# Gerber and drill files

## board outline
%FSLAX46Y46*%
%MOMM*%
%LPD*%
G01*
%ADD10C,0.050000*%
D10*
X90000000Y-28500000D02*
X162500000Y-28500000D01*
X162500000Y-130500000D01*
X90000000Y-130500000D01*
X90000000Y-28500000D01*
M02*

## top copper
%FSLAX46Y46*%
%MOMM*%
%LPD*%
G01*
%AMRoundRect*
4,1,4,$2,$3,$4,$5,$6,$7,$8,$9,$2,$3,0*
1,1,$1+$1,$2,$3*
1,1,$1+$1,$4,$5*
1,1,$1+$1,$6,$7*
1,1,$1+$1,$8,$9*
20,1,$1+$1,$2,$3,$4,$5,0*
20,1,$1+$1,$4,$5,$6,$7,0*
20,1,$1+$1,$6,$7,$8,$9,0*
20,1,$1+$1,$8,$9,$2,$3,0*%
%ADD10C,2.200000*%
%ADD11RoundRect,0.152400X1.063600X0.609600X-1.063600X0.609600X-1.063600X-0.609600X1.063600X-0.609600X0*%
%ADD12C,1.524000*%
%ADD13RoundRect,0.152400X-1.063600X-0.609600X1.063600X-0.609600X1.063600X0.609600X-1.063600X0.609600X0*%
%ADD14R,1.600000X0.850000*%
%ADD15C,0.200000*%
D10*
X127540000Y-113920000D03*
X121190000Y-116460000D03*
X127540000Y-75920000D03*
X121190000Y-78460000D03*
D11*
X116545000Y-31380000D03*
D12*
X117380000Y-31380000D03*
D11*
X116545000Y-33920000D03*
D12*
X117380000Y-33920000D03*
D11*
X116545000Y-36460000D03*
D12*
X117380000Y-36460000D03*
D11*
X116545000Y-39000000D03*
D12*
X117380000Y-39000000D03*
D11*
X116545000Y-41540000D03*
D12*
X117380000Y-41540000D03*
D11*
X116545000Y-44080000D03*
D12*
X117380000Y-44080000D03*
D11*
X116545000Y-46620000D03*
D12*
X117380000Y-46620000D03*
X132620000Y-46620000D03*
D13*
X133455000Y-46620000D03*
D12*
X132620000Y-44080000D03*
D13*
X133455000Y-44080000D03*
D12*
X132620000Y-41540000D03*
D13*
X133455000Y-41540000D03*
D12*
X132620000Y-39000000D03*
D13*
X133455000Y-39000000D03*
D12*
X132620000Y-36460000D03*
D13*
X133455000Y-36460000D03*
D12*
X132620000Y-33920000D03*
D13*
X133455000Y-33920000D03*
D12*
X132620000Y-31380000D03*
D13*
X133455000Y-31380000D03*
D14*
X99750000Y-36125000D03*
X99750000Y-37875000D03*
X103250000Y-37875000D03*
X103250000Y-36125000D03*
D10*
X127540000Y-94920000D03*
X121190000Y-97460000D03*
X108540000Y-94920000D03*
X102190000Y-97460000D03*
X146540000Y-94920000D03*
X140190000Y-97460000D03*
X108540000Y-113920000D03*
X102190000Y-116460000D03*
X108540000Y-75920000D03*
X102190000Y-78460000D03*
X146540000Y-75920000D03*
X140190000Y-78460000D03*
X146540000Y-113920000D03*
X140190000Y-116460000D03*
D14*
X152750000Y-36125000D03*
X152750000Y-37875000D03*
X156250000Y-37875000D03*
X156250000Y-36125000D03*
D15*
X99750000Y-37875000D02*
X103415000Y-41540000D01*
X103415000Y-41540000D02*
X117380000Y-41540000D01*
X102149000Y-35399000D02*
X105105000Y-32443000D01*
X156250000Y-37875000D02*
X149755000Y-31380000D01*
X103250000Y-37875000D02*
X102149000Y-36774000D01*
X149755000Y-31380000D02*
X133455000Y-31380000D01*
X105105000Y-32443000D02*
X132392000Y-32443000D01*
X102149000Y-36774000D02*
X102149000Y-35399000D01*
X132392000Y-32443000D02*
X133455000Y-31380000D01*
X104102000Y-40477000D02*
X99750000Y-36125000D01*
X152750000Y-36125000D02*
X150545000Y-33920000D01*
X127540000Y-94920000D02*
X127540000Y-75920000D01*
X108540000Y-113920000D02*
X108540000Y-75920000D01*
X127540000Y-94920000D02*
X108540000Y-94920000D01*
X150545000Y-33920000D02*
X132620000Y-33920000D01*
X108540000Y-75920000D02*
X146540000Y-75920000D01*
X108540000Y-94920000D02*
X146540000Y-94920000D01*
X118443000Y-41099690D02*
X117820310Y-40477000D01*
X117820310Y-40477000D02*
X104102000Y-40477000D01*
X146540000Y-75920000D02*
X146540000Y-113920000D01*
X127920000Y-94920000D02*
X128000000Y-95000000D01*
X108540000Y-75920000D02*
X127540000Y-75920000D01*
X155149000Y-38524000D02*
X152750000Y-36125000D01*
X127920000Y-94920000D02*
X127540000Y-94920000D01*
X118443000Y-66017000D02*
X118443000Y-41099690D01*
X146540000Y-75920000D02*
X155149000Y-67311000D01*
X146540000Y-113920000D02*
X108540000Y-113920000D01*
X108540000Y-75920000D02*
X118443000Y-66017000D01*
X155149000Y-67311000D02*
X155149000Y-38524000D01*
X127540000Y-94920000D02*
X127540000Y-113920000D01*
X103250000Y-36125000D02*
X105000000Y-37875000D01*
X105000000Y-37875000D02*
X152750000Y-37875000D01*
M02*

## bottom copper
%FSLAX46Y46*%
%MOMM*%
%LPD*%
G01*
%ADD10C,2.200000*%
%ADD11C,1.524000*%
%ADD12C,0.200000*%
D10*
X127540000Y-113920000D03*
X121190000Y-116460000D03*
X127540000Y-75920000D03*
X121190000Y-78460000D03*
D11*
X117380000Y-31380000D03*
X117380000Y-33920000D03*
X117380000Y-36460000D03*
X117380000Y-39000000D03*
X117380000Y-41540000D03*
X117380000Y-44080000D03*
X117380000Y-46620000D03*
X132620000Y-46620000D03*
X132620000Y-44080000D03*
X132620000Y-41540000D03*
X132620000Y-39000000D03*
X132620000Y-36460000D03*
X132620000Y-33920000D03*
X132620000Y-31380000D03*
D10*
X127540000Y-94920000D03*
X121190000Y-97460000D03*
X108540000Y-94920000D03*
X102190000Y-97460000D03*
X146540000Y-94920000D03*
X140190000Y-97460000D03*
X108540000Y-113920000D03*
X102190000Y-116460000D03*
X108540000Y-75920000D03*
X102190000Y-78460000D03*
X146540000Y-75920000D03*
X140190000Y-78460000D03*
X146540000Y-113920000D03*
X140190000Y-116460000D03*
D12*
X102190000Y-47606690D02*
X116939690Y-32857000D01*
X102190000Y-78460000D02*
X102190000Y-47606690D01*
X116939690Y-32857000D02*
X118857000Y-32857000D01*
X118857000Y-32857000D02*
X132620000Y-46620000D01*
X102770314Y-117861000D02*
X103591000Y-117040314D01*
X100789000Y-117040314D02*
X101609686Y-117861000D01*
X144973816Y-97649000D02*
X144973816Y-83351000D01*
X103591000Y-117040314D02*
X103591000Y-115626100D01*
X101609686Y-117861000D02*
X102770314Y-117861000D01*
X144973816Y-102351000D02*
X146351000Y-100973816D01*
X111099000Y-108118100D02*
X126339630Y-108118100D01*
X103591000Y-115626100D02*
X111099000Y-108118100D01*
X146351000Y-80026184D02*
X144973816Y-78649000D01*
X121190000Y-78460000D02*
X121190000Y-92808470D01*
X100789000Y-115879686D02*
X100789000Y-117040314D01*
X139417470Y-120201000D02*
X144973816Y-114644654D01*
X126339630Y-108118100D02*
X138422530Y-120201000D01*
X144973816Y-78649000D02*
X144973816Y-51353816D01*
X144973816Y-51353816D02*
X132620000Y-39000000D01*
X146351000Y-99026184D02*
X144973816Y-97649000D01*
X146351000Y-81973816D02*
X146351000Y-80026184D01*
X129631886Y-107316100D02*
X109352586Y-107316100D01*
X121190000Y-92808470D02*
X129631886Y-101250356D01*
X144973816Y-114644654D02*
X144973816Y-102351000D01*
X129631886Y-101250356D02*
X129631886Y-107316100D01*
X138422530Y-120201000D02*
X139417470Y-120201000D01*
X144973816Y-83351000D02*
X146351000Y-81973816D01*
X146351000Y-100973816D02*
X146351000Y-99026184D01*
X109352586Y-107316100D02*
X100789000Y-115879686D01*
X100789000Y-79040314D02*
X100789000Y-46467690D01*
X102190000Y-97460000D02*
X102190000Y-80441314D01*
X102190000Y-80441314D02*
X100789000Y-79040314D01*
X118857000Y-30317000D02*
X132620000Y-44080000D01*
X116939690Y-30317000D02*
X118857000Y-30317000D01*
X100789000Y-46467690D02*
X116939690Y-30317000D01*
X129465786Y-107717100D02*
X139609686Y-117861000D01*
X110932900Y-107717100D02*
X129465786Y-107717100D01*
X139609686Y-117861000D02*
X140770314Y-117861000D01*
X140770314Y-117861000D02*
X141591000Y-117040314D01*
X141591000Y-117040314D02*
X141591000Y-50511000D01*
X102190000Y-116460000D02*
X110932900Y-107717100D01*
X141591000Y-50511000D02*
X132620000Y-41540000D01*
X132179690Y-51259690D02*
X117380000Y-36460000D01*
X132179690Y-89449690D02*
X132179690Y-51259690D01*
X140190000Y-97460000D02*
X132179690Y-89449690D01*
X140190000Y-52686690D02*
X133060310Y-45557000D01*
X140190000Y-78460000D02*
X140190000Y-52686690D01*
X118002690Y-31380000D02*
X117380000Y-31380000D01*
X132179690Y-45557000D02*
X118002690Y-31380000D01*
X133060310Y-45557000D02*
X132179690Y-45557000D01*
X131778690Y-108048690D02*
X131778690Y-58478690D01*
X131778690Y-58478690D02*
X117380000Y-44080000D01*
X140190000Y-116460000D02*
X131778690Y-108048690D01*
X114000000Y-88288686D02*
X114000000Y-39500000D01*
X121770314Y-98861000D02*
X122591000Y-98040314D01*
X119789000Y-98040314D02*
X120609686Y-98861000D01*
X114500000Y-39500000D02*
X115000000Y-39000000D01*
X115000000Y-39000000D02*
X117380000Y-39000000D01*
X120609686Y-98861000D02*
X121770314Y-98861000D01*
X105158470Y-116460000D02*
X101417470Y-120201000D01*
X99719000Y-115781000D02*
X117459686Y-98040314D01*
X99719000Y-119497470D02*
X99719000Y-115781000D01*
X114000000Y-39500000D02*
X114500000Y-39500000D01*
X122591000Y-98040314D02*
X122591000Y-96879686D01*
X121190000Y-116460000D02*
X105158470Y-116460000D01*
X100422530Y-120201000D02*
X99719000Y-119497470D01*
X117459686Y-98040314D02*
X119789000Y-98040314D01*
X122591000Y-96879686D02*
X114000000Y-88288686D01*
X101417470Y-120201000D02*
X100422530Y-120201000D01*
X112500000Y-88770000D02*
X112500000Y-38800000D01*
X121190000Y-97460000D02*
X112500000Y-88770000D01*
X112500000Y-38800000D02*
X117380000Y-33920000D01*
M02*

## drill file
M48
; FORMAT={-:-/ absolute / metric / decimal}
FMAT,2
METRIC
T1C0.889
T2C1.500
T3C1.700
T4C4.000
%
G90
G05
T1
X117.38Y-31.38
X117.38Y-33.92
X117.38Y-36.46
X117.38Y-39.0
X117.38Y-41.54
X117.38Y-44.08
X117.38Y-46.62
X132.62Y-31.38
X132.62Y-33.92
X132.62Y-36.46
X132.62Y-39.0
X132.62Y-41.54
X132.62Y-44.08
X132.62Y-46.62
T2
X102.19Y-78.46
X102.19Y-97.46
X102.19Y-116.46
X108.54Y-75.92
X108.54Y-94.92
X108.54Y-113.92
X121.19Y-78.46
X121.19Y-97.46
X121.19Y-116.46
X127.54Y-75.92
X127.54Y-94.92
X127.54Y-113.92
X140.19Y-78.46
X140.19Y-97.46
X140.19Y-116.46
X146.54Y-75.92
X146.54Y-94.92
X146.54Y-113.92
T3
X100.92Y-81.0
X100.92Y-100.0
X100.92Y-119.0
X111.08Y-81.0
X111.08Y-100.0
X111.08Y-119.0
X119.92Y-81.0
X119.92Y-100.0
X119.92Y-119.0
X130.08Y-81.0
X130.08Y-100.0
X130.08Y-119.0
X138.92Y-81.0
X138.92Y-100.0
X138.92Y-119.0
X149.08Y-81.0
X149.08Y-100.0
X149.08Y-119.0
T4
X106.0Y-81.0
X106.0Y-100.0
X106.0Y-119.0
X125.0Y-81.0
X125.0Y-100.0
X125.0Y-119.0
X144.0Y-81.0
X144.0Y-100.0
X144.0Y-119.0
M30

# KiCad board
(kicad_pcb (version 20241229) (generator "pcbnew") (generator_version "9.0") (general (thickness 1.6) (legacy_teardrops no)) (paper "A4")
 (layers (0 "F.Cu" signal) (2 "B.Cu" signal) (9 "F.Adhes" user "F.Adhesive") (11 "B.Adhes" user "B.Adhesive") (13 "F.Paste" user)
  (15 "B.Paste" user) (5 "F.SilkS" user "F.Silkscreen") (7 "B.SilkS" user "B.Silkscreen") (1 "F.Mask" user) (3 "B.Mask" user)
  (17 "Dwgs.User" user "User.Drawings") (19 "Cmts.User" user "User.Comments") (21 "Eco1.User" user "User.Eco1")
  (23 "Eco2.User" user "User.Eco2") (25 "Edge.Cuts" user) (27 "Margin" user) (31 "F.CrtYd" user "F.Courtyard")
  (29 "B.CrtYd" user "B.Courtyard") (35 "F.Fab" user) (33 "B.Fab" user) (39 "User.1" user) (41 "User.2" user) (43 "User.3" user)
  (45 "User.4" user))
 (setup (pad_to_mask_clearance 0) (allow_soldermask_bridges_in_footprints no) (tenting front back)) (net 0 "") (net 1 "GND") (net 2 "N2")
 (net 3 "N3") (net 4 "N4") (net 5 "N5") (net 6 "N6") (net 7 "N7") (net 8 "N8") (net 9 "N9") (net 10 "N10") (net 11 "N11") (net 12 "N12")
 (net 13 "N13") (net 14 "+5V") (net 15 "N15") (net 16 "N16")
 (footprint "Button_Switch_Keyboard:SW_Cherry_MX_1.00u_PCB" (layer "F.Cu") (at 127.54 113.92)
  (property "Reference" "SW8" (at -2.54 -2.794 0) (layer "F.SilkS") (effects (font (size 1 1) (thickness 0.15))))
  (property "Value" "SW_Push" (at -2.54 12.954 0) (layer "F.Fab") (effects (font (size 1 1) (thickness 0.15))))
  (pad "" np_thru_hole circle (at -7.62 5.08) (size 1.7 1.7) (drill 1.7) (layers "*.Cu" "*.Mask"))
  (pad "" np_thru_hole circle (at -2.54 5.08) (size 4 4) (drill 4) (layers "*.Cu" "*.Mask"))
  (pad "" np_thru_hole circle (at 2.54 5.08) (size 1.7 1.7) (drill 1.7) (layers "*.Cu" "*.Mask"))
  (pad "1" thru_hole circle (at 0 0) (size 2.2 2.2) (drill 1.5) (layers "*.Cu" "*.Mask") (remove_unused_layers no) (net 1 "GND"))
  (pad "2" thru_hole circle (at -6.35 2.54) (size 2.2 2.2) (drill 1.5) (layers "*.Cu" "*.Mask") (remove_unused_layers no) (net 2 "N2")))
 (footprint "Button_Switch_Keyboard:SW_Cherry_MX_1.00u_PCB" (layer "F.Cu") (at 127.54 75.92)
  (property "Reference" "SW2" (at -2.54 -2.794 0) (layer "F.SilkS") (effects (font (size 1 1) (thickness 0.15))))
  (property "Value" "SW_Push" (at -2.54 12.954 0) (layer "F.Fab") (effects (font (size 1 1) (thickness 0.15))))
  (pad "" np_thru_hole circle (at -7.62 5.08) (size 1.7 1.7) (drill 1.7) (layers "*.Cu" "*.Mask"))
  (pad "" np_thru_hole circle (at -2.54 5.08) (size 4 4) (drill 4) (layers "*.Cu" "*.Mask"))
  (pad "" np_thru_hole circle (at 2.54 5.08) (size 1.7 1.7) (drill 1.7) (layers "*.Cu" "*.Mask"))
  (pad "1" thru_hole circle (at 0 0) (size 2.2 2.2) (drill 1.5) (layers "*.Cu" "*.Mask") (remove_unused_layers no) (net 1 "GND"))
  (pad "2" thru_hole circle (at -6.35 2.54) (size 2.2 2.2) (drill 1.5) (layers "*.Cu" "*.Mask") (remove_unused_layers no) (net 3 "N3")))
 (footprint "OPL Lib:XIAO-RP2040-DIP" (layer "F.Cu") (at 125 39)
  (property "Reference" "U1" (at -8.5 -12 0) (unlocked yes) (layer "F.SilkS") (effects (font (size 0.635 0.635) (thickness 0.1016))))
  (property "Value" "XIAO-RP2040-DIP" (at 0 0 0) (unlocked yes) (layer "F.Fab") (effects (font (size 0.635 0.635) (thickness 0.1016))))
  (pad "1" smd roundrect (at -8.455 -7.62 180) (size 2.432 1.524) (layers "F.Cu" "F.Mask") (roundrect_rratio 0.1) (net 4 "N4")
   (thermal_bridge_angle 45))
  (pad "1" thru_hole circle (at -7.62 -7.62 180) (size 1.524 1.524) (drill 0.889) (layers "*.Cu" "*.Mask") (remove_unused_layers no)
   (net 4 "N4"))
  (pad "2" smd roundrect (at -8.455 -5.08 180) (size 2.432 1.524) (layers "F.Cu" "F.Mask") (roundrect_rratio 0.1) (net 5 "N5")
   (thermal_bridge_angle 45))
  (pad "2" thru_hole circle (at -7.62 -5.08 180) (size 1.524 1.524) (drill 0.889) (layers "*.Cu" "*.Mask") (remove_unused_layers no)
   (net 5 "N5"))
  (pad "3" smd roundrect (at -8.455 -2.54 180) (size 2.432 1.524) (layers "F.Cu" "F.Mask") (roundrect_rratio 0.1) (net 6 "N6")
   (thermal_bridge_angle 45))
  (pad "3" thru_hole circle (at -7.62 -2.54 180) (size 1.524 1.524) (drill 0.889) (layers "*.Cu" "*.Mask") (remove_unused_layers no)
   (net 6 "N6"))
  (pad "4" smd roundrect (at -8.455 0 180) (size 2.432 1.524) (layers "F.Cu" "F.Mask") (roundrect_rratio 0.1) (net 2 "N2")
   (thermal_bridge_angle 45))
  (pad "4" thru_hole circle (at -7.62 0 180) (size 1.524 1.524) (drill 0.889) (layers "*.Cu" "*.Mask") (remove_unused_layers no)
   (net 2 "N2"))
  (pad "5" smd roundrect (at -8.455 2.54 180) (size 2.432 1.524) (layers "F.Cu" "F.Mask") (roundrect_rratio 0.1) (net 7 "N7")
   (thermal_bridge_angle 45))
  (pad "5" thru_hole circle (at -7.62 2.54 180) (size 1.524 1.524) (drill 0.889) (layers "*.Cu" "*.Mask") (remove_unused_layers no)
   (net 7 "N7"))
  (pad "6" smd roundrect (at -8.455 5.08 180) (size 2.432 1.524) (layers "F.Cu" "F.Mask") (roundrect_rratio 0.1) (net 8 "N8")
   (thermal_bridge_angle 45))
  (pad "6" thru_hole circle (at -7.62 5.08 180) (size 1.524 1.524) (drill 0.889) (layers "*.Cu" "*.Mask") (remove_unused_layers no)
   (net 8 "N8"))
  (pad "7" smd roundrect (at -8.455 7.62 180) (size 2.432 1.524) (layers "F.Cu" "F.Mask") (roundrect_rratio 0.1) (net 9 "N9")
   (thermal_bridge_angle 45))
  (pad "7" thru_hole circle (at -7.62 7.62 180) (size 1.524 1.524) (drill 0.889) (layers "*.Cu" "*.Mask") (remove_unused_layers no)
   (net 9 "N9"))
  (pad "8" thru_hole circle (at 7.62 7.62) (size 1.524 1.524) (drill 0.889) (layers "*.Cu" "*.Mask") (remove_unused_layers no)
   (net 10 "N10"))
  (pad "8" smd roundrect (at 8.455 7.62) (size 2.432 1.524) (layers "F.Cu" "F.Mask") (roundrect_rratio 0.1) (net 10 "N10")
   (thermal_bridge_angle 45))
  (pad "9" thru_hole circle (at 7.62 5.08) (size 1.524 1.524) (drill 0.889) (layers "*.Cu" "*.Mask") (remove_unused_layers no)
   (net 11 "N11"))
  (pad "9" smd roundrect (at 8.455 5.08) (size 2.432 1.524) (layers "F.Cu" "F.Mask") (roundrect_rratio 0.1) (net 11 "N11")
   (thermal_bridge_angle 45))
  (pad "10" thru_hole circle (at 7.62 2.54) (size 1.524 1.524) (drill 0.889) (layers "*.Cu" "*.Mask") (remove_unused_layers no)
   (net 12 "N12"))
  (pad "10" smd roundrect (at 8.455 2.54) (size 2.432 1.524) (layers "F.Cu" "F.Mask") (roundrect_rratio 0.1) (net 12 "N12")
   (thermal_bridge_angle 45))
  (pad "11" thru_hole circle (at 7.62 0) (size 1.524 1.524) (drill 0.889) (layers "*.Cu" "*.Mask") (remove_unused_layers no) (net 3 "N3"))
  (pad "11" smd roundrect (at 8.455 0) (size 2.432 1.524) (layers "F.Cu" "F.Mask") (roundrect_rratio 0.1) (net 3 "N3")
   (thermal_bridge_angle 45))
  (pad "12" thru_hole circle (at 7.62 -2.54) (size 1.524 1.524) (drill 0.889) (layers "*.Cu" "*.Mask") (remove_unused_layers no)
   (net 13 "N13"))
  (pad "12" smd roundrect (at 8.455 -2.54) (size 2.432 1.524) (layers "F.Cu" "F.Mask") (roundrect_rratio 0.1) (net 13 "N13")
   (thermal_bridge_angle 45))
  (pad "13" thru_hole circle (at 7.62 -5.08) (size 1.524 1.524) (drill 0.889) (layers "*.Cu" "*.Mask") (remove_unused_layers no)
   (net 1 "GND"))
  (pad "13" smd roundrect (at 8.455 -5.08) (size 2.432 1.524) (layers "F.Cu" "F.Mask") (roundrect_rratio 0.1) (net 1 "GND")
   (thermal_bridge_angle 45))
  (pad "14" thru_hole circle (at 7.62 -7.62) (size 1.524 1.524) (drill 0.889) (layers "*.Cu" "*.Mask") (remove_unused_layers no)
   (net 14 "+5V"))
  (pad "14" smd roundrect (at 8.455 -7.62) (size 2.432 1.524) (layers "F.Cu" "F.Mask") (roundrect_rratio 0.1) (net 14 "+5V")
   (thermal_bridge_angle 45)))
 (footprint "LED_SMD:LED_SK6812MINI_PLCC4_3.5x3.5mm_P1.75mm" (layer "F.Cu") (at 101.5 37)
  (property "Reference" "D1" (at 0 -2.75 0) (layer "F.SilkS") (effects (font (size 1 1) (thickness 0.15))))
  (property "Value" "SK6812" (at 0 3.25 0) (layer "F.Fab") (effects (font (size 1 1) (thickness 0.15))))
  (pad "1" smd rect (at -1.75 -0.875) (size 1.6 0.85) (layers "F.Cu" "F.Mask" "F.Paste") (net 1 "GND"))
  (pad "2" smd rect (at -1.75 0.875) (size 1.6 0.85) (layers "F.Cu" "F.Mask" "F.Paste") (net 7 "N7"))
  (pad "3" smd rect (at 1.75 0.875) (size 1.6 0.85) (layers "F.Cu" "F.Mask" "F.Paste") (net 14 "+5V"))
  (pad "4" smd rect (at 1.75 -0.875) (size 1.6 0.85) (layers "F.Cu" "F.Mask" "F.Paste") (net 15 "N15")))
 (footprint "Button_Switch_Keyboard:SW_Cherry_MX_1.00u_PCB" (layer "F.Cu") (at 127.54 94.92)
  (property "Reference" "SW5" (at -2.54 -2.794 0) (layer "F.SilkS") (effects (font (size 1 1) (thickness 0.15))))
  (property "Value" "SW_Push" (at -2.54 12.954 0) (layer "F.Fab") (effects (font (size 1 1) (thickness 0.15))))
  (pad "" np_thru_hole circle (at -7.62 5.08) (size 1.7 1.7) (drill 1.7) (layers "*.Cu" "*.Mask"))
  (pad "" np_thru_hole circle (at -2.54 5.08) (size 4 4) (drill 4) (layers "*.Cu" "*.Mask"))
  (pad "" np_thru_hole circle (at 2.54 5.08) (size 1.7 1.7) (drill 1.7) (layers "*.Cu" "*.Mask"))
  (pad "1" thru_hole circle (at 0 0) (size 2.2 2.2) (drill 1.5) (layers "*.Cu" "*.Mask") (remove_unused_layers no) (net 1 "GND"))
  (pad "2" thru_hole circle (at -6.35 2.54) (size 2.2 2.2) (drill 1.5) (layers "*.Cu" "*.Mask") (remove_unused_layers no) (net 5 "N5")))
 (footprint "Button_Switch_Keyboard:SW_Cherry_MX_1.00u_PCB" (layer "F.Cu") (at 108.54 94.92)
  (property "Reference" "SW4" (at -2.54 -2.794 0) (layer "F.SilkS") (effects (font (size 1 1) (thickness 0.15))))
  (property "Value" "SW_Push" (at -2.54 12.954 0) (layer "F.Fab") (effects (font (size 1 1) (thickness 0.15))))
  (pad "" np_thru_hole circle (at -7.62 5.08) (size 1.7 1.7) (drill 1.7) (layers "*.Cu" "*.Mask"))
  (pad "" np_thru_hole circle (at -2.54 5.08) (size 4 4) (drill 4) (layers "*.Cu" "*.Mask"))
  (pad "" np_thru_hole circle (at 2.54 5.08) (size 1.7 1.7) (drill 1.7) (layers "*.Cu" "*.Mask"))
  (pad "1" thru_hole circle (at 0 0) (size 2.2 2.2) (drill 1.5) (layers "*.Cu" "*.Mask") (remove_unused_layers no) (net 1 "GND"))
  (pad "2" thru_hole circle (at -6.35 2.54) (size 2.2 2.2) (drill 1.5) (layers "*.Cu" "*.Mask") (remove_unused_layers no) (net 11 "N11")))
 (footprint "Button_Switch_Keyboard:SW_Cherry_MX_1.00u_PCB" (layer "F.Cu") (at 146.54 94.92)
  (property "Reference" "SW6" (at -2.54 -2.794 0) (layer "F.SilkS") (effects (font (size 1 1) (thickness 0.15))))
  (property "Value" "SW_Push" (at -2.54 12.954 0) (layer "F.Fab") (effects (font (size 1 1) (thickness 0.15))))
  (pad "" np_thru_hole circle (at -7.62 5.08) (size 1.7 1.7) (drill 1.7) (layers "*.Cu" "*.Mask"))
  (pad "" np_thru_hole circle (at -2.54 5.08) (size 4 4) (drill 4) (layers "*.Cu" "*.Mask"))
  (pad "" np_thru_hole circle (at 2.54 5.08) (size 1.7 1.7) (drill 1.7) (layers "*.Cu" "*.Mask"))
  (pad "1" thru_hole circle (at 0 0) (size 2.2 2.2) (drill 1.5) (layers "*.Cu" "*.Mask") (remove_unused_layers no) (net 1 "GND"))
  (pad "2" thru_hole circle (at -6.35 2.54) (size 2.2 2.2) (drill 1.5) (layers "*.Cu" "*.Mask") (remove_unused_layers no) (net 6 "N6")))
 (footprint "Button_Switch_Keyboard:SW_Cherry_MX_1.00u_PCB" (layer "F.Cu") (at 108.54 113.92)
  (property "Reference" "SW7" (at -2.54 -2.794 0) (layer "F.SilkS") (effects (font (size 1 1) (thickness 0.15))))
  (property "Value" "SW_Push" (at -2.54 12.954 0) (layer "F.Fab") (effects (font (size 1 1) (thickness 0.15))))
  (pad "" np_thru_hole circle (at -7.62 5.08) (size 1.7 1.7) (drill 1.7) (layers "*.Cu" "*.Mask"))
  (pad "" np_thru_hole circle (at -2.54 5.08) (size 4 4) (drill 4) (layers "*.Cu" "*.Mask"))
  (pad "" np_thru_hole circle (at 2.54 5.08) (size 1.7 1.7) (drill 1.7) (layers "*.Cu" "*.Mask"))
  (pad "1" thru_hole circle (at 0 0) (size 2.2 2.2) (drill 1.5) (layers "*.Cu" "*.Mask") (remove_unused_layers no) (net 1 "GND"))
  (pad "2" thru_hole circle (at -6.35 2.54) (size 2.2 2.2) (drill 1.5) (layers "*.Cu" "*.Mask") (remove_unused_layers no) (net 12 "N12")))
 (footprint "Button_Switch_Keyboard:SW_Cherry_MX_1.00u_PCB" (layer "F.Cu") (at 108.54 75.92)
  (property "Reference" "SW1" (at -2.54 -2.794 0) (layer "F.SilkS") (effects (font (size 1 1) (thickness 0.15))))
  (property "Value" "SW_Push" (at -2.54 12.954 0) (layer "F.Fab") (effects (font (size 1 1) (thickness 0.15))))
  (pad "" np_thru_hole circle (at -7.62 5.08) (size 1.7 1.7) (drill 1.7) (layers "*.Cu" "*.Mask"))
  (pad "" np_thru_hole circle (at -2.54 5.08) (size 4 4) (drill 4) (layers "*.Cu" "*.Mask"))
  (pad "" np_thru_hole circle (at 2.54 5.08) (size 1.7 1.7) (drill 1.7) (layers "*.Cu" "*.Mask"))
  (pad "1" thru_hole circle (at 0 0) (size 2.2 2.2) (drill 1.5) (layers "*.Cu" "*.Mask") (remove_unused_layers no) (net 1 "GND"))
  (pad "2" thru_hole circle (at -6.35 2.54) (size 2.2 2.2) (drill 1.5) (layers "*.Cu" "*.Mask") (remove_unused_layers no) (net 10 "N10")))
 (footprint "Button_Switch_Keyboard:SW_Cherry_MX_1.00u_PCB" (layer "F.Cu") (at 146.54 75.92)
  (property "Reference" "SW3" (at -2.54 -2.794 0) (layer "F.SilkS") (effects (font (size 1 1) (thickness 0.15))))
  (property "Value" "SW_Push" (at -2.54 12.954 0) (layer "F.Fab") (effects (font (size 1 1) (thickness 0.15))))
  (pad "" np_thru_hole circle (at -7.62 5.08) (size 1.7 1.7) (drill 1.7) (layers "*.Cu" "*.Mask"))
  (pad "" np_thru_hole circle (at -2.54 5.08) (size 4 4) (drill 4) (layers "*.Cu" "*.Mask"))
  (pad "" np_thru_hole circle (at 2.54 5.08) (size 1.7 1.7) (drill 1.7) (layers "*.Cu" "*.Mask"))
  (pad "1" thru_hole circle (at 0 0) (size 2.2 2.2) (drill 1.5) (layers "*.Cu" "*.Mask") (remove_unused_layers no) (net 1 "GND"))
  (pad "2" thru_hole circle (at -6.35 2.54) (size 2.2 2.2) (drill 1.5) (layers "*.Cu" "*.Mask") (remove_unused_layers no) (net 4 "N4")))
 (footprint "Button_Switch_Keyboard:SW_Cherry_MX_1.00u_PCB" (layer "F.Cu") (at 146.54 113.92)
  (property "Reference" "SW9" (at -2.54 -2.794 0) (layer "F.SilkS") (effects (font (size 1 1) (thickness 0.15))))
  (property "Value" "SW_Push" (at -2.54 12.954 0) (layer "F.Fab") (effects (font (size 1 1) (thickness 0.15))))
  (pad "" np_thru_hole circle (at -7.62 5.08) (size 1.7 1.7) (drill 1.7) (layers "*.Cu" "*.Mask"))
  (pad "" np_thru_hole circle (at -2.54 5.08) (size 4 4) (drill 4) (layers "*.Cu" "*.Mask"))
  (pad "" np_thru_hole circle (at 2.54 5.08) (size 1.7 1.7) (drill 1.7) (layers "*.Cu" "*.Mask"))
  (pad "1" thru_hole circle (at 0 0) (size 2.2 2.2) (drill 1.5) (layers "*.Cu" "*.Mask") (remove_unused_layers no) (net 1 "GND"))
  (pad "2" thru_hole circle (at -6.35 2.54) (size 2.2 2.2) (drill 1.5) (layers "*.Cu" "*.Mask") (remove_unused_layers no) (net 8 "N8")))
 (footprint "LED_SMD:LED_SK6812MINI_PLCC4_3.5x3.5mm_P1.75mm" (layer "F.Cu") (at 154.5 37)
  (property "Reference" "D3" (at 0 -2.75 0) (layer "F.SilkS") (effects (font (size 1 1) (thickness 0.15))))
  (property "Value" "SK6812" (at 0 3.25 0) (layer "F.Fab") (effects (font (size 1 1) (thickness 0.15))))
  (pad "1" smd rect (at -1.75 -0.875) (size 1.6 0.85) (layers "F.Cu" "F.Mask" "F.Paste") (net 1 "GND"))
  (pad "2" smd rect (at -1.75 0.875) (size 1.6 0.85) (layers "F.Cu" "F.Mask" "F.Paste") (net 15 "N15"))
  (pad "3" smd rect (at 1.75 0.875) (size 1.6 0.85) (layers "F.Cu" "F.Mask" "F.Paste") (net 14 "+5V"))
  (pad "4" smd rect (at 1.75 -0.875) (size 1.6 0.85) (layers "F.Cu" "F.Mask" "F.Paste") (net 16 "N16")))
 (gr_rect (start 90 28.5) (end 162.5 130.5) (stroke (width 0.05) (type default)) (fill no) (layer "Edge.Cuts"))
 (segment (start 99.75 37.875) (end 103.415 41.54) (width 0.2) (layer "F.Cu") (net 7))
 (segment (start 103.415 41.54) (end 117.38 41.54) (width 0.2) (layer "F.Cu") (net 7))
 (segment (start 102.149 35.399) (end 105.105 32.443) (width 0.2) (layer "F.Cu") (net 14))
 (segment (start 156.25 37.875) (end 149.755 31.38) (width 0.2) (layer "F.Cu") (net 14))
 (segment (start 103.25 37.875) (end 102.149 36.774) (width 0.2) (layer "F.Cu") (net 14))
 (segment (start 149.755 31.38) (end 133.455 31.38) (width 0.2) (layer "F.Cu") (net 14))
 (segment (start 105.105 32.443) (end 132.392 32.443) (width 0.2) (layer "F.Cu") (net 14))
 (segment (start 102.149 36.774) (end 102.149 35.399) (width 0.2) (layer "F.Cu") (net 14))
 (segment (start 132.392 32.443) (end 133.455 31.38) (width 0.2) (layer "F.Cu") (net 14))
 (segment (start 104.102 40.477) (end 99.75 36.125) (width 0.2) (layer "F.Cu") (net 1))
 (segment (start 152.75 36.125) (end 150.545 33.92) (width 0.2) (layer "F.Cu") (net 1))
 (segment (start 127.54 94.92) (end 127.54 75.92) (width 0.2) (layer "F.Cu") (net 1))
 (segment (start 108.54 113.92) (end 108.54 75.92) (width 0.2) (layer "F.Cu") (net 1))
 (segment (start 127.54 94.92) (end 108.54 94.92) (width 0.2) (layer "F.Cu") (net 1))
 (segment (start 150.545 33.92) (end 132.62 33.92) (width 0.2) (layer "F.Cu") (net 1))
 (segment (start 108.54 75.92) (end 146.54 75.92) (width 0.2) (layer "F.Cu") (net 1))
 (segment (start 108.54 94.92) (end 146.54 94.92) (width 0.2) (layer "F.Cu") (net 1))
 (segment (start 118.443 41.09969) (end 117.82031 40.477) (width 0.2) (layer "F.Cu") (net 1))
 (segment (start 117.82031 40.477) (end 104.102 40.477) (width 0.2) (layer "F.Cu") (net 1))
 (segment (start 146.54 75.92) (end 146.54 113.92) (width 0.2) (layer "F.Cu") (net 1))
 (segment (start 127.92 94.92) (end 128 95) (width 0.2) (layer "F.Cu") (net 1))
 (segment (start 108.54 75.92) (end 127.54 75.92) (width 0.2) (layer "F.Cu") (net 1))
 (segment (start 155.149 38.524) (end 152.75 36.125) (width 0.2) (layer "F.Cu") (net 1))
 (segment (start 127.92 94.92) (end 127.54 94.92) (width 0.2) (layer "F.Cu") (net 1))
 (segment (start 118.443 66.017) (end 118.443 41.09969) (width 0.2) (layer "F.Cu") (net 1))
 (segment (start 146.54 75.92) (end 155.149 67.311) (width 0.2) (layer "F.Cu") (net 1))
 (segment (start 146.54 113.92) (end 108.54 113.92) (width 0.2) (layer "F.Cu") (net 1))
 (segment (start 108.54 75.92) (end 118.443 66.017) (width 0.2) (layer "F.Cu") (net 1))
 (segment (start 155.149 67.311) (end 155.149 38.524) (width 0.2) (layer "F.Cu") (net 1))
 (segment (start 127.54 94.92) (end 127.54 113.92) (width 0.2) (layer "F.Cu") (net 1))
 (segment (start 103.25 36.125) (end 105 37.875) (width 0.2) (layer "F.Cu") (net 15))
 (segment (start 105 37.875) (end 152.75 37.875) (width 0.2) (layer "F.Cu") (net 15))
 (segment (start 102.19 47.60669) (end 116.93969 32.857) (width 0.2) (layer "B.Cu") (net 10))
 (segment (start 102.19 78.46) (end 102.19 47.60669) (width 0.2) (layer "B.Cu") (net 10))
 (segment (start 116.93969 32.857) (end 118.857 32.857) (width 0.2) (layer "B.Cu") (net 10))
 (segment (start 118.857 32.857) (end 132.62 46.62) (width 0.2) (layer "B.Cu") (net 10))
 (segment (start 102.770314 117.861) (end 103.591 117.040314) (width 0.2) (layer "B.Cu") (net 3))
 (segment (start 100.789 117.040314) (end 101.609686 117.861) (width 0.2) (layer "B.Cu") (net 3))
 (segment (start 144.973816 97.649) (end 144.973816 83.351) (width 0.2) (layer "B.Cu") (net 3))
 (segment (start 103.591 117.040314) (end 103.591 115.6261) (width 0.2) (layer "B.Cu") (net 3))
 (segment (start 101.609686 117.861) (end 102.770314 117.861) (width 0.2) (layer "B.Cu") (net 3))
 (segment (start 144.973816 102.351) (end 146.351 100.973816) (width 0.2) (layer "B.Cu") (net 3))
 (segment (start 111.099 108.1181) (end 126.33963 108.1181) (width 0.2) (layer "B.Cu") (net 3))
 (segment (start 103.591 115.6261) (end 111.099 108.1181) (width 0.2) (layer "B.Cu") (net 3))
 (segment (start 146.351 80.026184) (end 144.973816 78.649) (width 0.2) (layer "B.Cu") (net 3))
 (segment (start 121.19 78.46) (end 121.19 92.80847) (width 0.2) (layer "B.Cu") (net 3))
 (segment (start 100.789 115.879686) (end 100.789 117.040314) (width 0.2) (layer "B.Cu") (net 3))
 (segment (start 139.41747 120.201) (end 144.973816 114.644654) (width 0.2) (layer "B.Cu") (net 3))
 (segment (start 126.33963 108.1181) (end 138.42253 120.201) (width 0.2) (layer "B.Cu") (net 3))
 (segment (start 144.973816 78.649) (end 144.973816 51.353816) (width 0.2) (layer "B.Cu") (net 3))
 (segment (start 144.973816 51.353816) (end 132.62 39) (width 0.2) (layer "B.Cu") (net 3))
 (segment (start 146.351 99.026184) (end 144.973816 97.649) (width 0.2) (layer "B.Cu") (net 3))
 (segment (start 146.351 81.973816) (end 146.351 80.026184) (width 0.2) (layer "B.Cu") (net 3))
 (segment (start 129.631886 107.3161) (end 109.352586 107.3161) (width 0.2) (layer "B.Cu") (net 3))
 (segment (start 121.19 92.80847) (end 129.631886 101.250356) (width 0.2) (layer "B.Cu") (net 3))
 (segment (start 144.973816 114.644654) (end 144.973816 102.351) (width 0.2) (layer "B.Cu") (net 3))
 (segment (start 129.631886 101.250356) (end 129.631886 107.3161) (width 0.2) (layer "B.Cu") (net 3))
 (segment (start 138.42253 120.201) (end 139.41747 120.201) (width 0.2) (layer "B.Cu") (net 3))
 (segment (start 144.973816 83.351) (end 146.351 81.973816) (width 0.2) (layer "B.Cu") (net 3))
 (segment (start 146.351 100.973816) (end 146.351 99.026184) (width 0.2) (layer "B.Cu") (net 3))
 (segment (start 109.352586 107.3161) (end 100.789 115.879686) (width 0.2) (layer "B.Cu") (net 3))
 (segment (start 100.789 79.040314) (end 100.789 46.46769) (width 0.2) (layer "B.Cu") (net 11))
 (segment (start 102.19 97.46) (end 102.19 80.441314) (width 0.2) (layer "B.Cu") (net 11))
 (segment (start 102.19 80.441314) (end 100.789 79.040314) (width 0.2) (layer "B.Cu") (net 11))
 (segment (start 118.857 30.317) (end 132.62 44.08) (width 0.2) (layer "B.Cu") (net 11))
 (segment (start 116.93969 30.317) (end 118.857 30.317) (width 0.2) (layer "B.Cu") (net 11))
 (segment (start 100.789 46.46769) (end 116.93969 30.317) (width 0.2) (layer "B.Cu") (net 11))
 (segment (start 129.465786 107.7171) (end 139.609686 117.861) (width 0.2) (layer "B.Cu") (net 12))
 (segment (start 110.9329 107.7171) (end 129.465786 107.7171) (width 0.2) (layer "B.Cu") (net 12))
 (segment (start 139.609686 117.861) (end 140.770314 117.861) (width 0.2) (layer "B.Cu") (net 12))
 (segment (start 140.770314 117.861) (end 141.591 117.040314) (width 0.2) (layer "B.Cu") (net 12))
 (segment (start 141.591 117.040314) (end 141.591 50.511) (width 0.2) (layer "B.Cu") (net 12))
 (segment (start 102.19 116.46) (end 110.9329 107.7171) (width 0.2) (layer "B.Cu") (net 12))
 (segment (start 141.591 50.511) (end 132.62 41.54) (width 0.2) (layer "B.Cu") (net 12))
 (segment (start 132.17969 51.25969) (end 117.38 36.46) (width 0.2) (layer "B.Cu") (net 6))
 (segment (start 132.17969 89.44969) (end 132.17969 51.25969) (width 0.2) (layer "B.Cu") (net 6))
 (segment (start 140.19 97.46) (end 132.17969 89.44969) (width 0.2) (layer "B.Cu") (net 6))
 (segment (start 140.19 52.68669) (end 133.06031 45.557) (width 0.2) (layer "B.Cu") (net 4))
 (segment (start 140.19 78.46) (end 140.19 52.68669) (width 0.2) (layer "B.Cu") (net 4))
 (segment (start 118.00269 31.38) (end 117.38 31.38) (width 0.2) (layer "B.Cu") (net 4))
 (segment (start 132.17969 45.557) (end 118.00269 31.38) (width 0.2) (layer "B.Cu") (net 4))
 (segment (start 133.06031 45.557) (end 132.17969 45.557) (width 0.2) (layer "B.Cu") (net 4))
 (segment (start 131.77869 108.04869) (end 131.77869 58.47869) (width 0.2) (layer "B.Cu") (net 8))
 (segment (start 131.77869 58.47869) (end 117.38 44.08) (width 0.2) (layer "B.Cu") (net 8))
 (segment (start 140.19 116.46) (end 131.77869 108.04869) (width 0.2) (layer "B.Cu") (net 8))
 (segment (start 114 88.288686) (end 114 39.5) (width 0.2) (layer "B.Cu") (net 2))
 (segment (start 121.770314 98.861) (end 122.591 98.040314) (width 0.2) (layer "B.Cu") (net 2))
 (segment (start 119.789 98.040314) (end 120.609686 98.861) (width 0.2) (layer "B.Cu") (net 2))
 (segment (start 114.5 39.5) (end 115 39) (width 0.2) (layer "B.Cu") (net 2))
 (segment (start 115 39) (end 117.38 39) (width 0.2) (layer "B.Cu") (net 2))
 (segment (start 120.609686 98.861) (end 121.770314 98.861) (width 0.2) (layer "B.Cu") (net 2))
 (segment (start 105.15847 116.46) (end 101.41747 120.201) (width 0.2) (layer "B.Cu") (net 2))
 (segment (start 99.719 115.781) (end 117.459686 98.040314) (width 0.2) (layer "B.Cu") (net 2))
 (segment (start 99.719 119.49747) (end 99.719 115.781) (width 0.2) (layer "B.Cu") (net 2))
 (segment (start 114 39.5) (end 114.5 39.5) (width 0.2) (layer "B.Cu") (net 2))
 (segment (start 122.591 98.040314) (end 122.591 96.879686) (width 0.2) (layer "B.Cu") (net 2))
 (segment (start 121.19 116.46) (end 105.15847 116.46) (width 0.2) (layer "B.Cu") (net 2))
 (segment (start 100.42253 120.201) (end 99.719 119.49747) (width 0.2) (layer "B.Cu") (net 2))
 (segment (start 117.459686 98.040314) (end 119.789 98.040314) (width 0.2) (layer "B.Cu") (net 2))
 (segment (start 122.591 96.879686) (end 114 88.288686) (width 0.2) (layer "B.Cu") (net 2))
 (segment (start 101.41747 120.201) (end 100.42253 120.201) (width 0.2) (layer "B.Cu") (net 2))
 (segment (start 112.5 88.77) (end 112.5 38.8) (width 0.2) (layer "B.Cu") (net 5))
 (segment (start 121.19 97.46) (end 112.5 88.77) (width 0.2) (layer "B.Cu") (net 5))
 (segment (start 112.5 38.8) (end 117.38 33.92) (width 0.2) (layer "B.Cu") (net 5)))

